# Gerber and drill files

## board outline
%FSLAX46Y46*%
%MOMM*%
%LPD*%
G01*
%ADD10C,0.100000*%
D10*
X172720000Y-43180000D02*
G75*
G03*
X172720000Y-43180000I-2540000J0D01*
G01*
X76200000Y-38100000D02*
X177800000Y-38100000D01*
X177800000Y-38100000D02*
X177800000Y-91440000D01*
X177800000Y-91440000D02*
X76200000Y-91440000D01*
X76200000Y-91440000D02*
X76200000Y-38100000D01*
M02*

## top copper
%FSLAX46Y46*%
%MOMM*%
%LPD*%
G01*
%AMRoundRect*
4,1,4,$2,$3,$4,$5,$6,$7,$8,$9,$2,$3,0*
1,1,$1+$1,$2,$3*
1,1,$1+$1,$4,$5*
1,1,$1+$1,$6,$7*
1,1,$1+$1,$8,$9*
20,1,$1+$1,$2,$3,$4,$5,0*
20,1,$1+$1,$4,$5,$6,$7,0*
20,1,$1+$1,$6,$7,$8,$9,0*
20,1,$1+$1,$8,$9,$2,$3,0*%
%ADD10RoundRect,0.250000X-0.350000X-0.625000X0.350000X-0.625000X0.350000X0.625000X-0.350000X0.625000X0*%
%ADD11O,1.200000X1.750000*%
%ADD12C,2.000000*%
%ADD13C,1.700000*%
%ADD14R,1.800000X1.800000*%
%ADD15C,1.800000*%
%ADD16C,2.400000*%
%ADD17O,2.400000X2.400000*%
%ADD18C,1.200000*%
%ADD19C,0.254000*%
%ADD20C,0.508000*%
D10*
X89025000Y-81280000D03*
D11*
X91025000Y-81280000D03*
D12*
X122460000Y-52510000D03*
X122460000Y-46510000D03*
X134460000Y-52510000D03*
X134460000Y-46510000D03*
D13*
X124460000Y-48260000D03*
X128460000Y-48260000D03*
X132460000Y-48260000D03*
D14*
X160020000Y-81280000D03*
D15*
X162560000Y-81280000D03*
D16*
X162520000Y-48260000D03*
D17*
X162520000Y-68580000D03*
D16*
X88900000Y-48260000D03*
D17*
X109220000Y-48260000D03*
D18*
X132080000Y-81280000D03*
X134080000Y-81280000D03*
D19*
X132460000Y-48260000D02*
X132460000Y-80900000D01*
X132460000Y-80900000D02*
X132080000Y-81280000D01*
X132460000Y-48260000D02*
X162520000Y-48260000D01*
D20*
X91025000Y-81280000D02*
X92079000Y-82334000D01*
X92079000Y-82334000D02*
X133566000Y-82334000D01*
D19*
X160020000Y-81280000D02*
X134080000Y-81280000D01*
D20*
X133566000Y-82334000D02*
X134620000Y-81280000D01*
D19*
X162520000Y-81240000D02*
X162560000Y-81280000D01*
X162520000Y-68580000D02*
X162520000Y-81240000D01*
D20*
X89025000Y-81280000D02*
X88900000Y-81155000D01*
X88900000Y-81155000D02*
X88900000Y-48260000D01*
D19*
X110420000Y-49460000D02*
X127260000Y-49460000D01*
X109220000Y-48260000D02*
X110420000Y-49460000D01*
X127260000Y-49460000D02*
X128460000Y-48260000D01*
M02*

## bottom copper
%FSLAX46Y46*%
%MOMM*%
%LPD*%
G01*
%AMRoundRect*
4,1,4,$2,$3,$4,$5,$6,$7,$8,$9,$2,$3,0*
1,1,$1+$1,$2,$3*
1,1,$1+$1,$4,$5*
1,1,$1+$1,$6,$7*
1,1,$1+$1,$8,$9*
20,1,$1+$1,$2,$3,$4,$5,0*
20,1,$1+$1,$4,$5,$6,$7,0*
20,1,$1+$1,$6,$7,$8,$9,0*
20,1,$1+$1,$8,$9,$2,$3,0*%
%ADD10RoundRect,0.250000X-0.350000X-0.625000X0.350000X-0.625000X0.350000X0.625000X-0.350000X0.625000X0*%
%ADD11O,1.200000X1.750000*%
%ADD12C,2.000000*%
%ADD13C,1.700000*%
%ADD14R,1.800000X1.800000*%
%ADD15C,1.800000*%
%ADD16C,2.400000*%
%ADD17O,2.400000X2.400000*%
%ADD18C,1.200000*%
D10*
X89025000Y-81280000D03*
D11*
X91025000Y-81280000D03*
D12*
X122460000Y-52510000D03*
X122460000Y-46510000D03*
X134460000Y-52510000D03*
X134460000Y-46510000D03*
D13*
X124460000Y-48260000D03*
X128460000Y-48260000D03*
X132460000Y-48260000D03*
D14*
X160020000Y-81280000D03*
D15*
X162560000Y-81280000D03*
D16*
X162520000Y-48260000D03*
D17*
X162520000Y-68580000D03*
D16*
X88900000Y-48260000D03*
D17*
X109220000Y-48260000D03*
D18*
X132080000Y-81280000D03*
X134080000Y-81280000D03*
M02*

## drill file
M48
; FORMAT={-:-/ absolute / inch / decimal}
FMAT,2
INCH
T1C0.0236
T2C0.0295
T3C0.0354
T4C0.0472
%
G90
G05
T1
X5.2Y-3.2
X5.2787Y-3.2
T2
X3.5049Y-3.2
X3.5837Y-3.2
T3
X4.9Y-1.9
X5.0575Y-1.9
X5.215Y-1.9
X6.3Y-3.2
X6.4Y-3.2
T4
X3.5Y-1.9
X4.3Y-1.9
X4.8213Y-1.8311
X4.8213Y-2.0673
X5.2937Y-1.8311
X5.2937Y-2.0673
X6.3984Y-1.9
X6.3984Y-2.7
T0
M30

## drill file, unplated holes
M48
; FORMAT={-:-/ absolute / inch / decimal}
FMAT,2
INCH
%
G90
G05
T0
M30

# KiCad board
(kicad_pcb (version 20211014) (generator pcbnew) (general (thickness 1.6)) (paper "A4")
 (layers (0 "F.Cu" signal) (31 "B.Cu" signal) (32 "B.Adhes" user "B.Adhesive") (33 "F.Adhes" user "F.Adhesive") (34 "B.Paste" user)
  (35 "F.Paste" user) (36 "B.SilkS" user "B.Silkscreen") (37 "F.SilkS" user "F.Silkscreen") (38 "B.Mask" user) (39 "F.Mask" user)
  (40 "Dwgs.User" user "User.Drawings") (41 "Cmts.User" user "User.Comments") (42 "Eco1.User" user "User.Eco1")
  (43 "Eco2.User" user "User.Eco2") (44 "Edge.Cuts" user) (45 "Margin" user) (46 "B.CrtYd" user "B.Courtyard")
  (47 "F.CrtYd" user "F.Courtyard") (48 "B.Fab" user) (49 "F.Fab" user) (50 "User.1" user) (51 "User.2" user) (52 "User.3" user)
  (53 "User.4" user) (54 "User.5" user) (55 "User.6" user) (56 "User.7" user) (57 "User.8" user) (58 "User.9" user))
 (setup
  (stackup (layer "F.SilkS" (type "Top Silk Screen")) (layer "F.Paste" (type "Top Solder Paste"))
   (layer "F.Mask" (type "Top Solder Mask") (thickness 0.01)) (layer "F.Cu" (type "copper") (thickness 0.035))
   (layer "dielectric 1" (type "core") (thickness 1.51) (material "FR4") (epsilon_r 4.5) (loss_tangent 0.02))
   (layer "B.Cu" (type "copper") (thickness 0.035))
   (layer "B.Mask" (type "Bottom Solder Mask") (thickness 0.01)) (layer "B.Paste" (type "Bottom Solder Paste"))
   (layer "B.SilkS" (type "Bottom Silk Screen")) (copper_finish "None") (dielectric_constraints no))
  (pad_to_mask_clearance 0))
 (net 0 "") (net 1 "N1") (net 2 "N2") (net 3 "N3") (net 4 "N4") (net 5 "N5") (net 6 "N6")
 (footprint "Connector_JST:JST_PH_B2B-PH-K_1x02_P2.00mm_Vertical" (layer "F.Cu") (at 89.025 81.28)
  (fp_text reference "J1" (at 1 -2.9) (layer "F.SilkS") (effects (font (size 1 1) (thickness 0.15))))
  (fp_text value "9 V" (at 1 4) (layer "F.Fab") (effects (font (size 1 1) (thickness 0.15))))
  (pad "1" thru_hole roundrect (at 0 0) (size 1.2 1.75) (drill 0.75) (layers *.Cu *.Mask) (roundrect_rratio 0.2083333333) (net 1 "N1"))
  (pad "2" thru_hole oval (at 2 0) (size 1.2 1.75) (drill 0.75) (layers *.Cu *.Mask) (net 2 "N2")))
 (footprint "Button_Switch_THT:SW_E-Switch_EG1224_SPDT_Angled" (layer "F.Cu") (at 124.46 48.26)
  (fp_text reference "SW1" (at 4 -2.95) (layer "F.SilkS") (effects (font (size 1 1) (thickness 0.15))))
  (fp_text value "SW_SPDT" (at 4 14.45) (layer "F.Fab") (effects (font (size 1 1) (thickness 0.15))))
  (pad "" thru_hole circle (at -2 4.25) (size 2 2) (drill 1.2) (layers *.Cu *.Mask))
  (pad "" thru_hole circle (at -2 -1.75) (size 2 2) (drill 1.2) (layers *.Cu *.Mask))
  (pad "" thru_hole circle (at 10 4.25) (size 2 2) (drill 1.2) (layers *.Cu *.Mask))
  (pad "" thru_hole circle (at 10 -1.75) (size 2 2) (drill 1.2) (layers *.Cu *.Mask))
  (pad "1" thru_hole circle (at 0 0) (size 1.7 1.7) (drill 0.9) (layers *.Cu *.Mask) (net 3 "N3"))
  (pad "2" thru_hole circle (at 4 0) (size 1.7 1.7) (drill 0.9) (layers *.Cu *.Mask) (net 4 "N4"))
  (pad "3" thru_hole circle (at 8 0) (size 1.7 1.7) (drill 0.9) (layers *.Cu *.Mask) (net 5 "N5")))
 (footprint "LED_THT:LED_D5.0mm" (layer "F.Cu") (at 160.02 81.28)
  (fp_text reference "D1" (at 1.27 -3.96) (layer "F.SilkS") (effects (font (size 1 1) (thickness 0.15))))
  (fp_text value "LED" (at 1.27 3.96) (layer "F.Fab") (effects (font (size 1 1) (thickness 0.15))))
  (pad "1" thru_hole rect (at 0 0) (size 1.8 1.8) (drill 0.9) (layers *.Cu *.Mask) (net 2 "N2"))
  (pad "2" thru_hole circle (at 2.54 0) (size 1.8 1.8) (drill 0.9) (layers *.Cu *.Mask) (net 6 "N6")))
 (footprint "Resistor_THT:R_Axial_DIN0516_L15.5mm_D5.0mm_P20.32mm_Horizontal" (layer "F.Cu") (at 162.52 48.26 -90)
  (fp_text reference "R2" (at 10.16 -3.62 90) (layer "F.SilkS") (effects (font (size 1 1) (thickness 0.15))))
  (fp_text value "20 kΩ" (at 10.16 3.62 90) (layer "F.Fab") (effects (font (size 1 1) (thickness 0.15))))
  (pad "1" thru_hole circle (at 0 0 270) (size 2.4 2.4) (drill 1.2) (layers *.Cu *.Mask) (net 5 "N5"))
  (pad "2" thru_hole oval (at 20.32 0 270) (size 2.4 2.4) (drill 1.2) (layers *.Cu *.Mask) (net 6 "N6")))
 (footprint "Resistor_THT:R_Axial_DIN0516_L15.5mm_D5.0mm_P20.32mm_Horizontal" (layer "F.Cu") (at 88.9 48.26)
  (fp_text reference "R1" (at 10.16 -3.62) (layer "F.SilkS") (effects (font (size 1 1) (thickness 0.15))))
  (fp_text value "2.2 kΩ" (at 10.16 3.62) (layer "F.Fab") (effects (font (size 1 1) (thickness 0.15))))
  (pad "1" thru_hole circle (at 0 0) (size 2.4 2.4) (drill 1.2) (layers *.Cu *.Mask) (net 1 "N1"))
  (pad "2" thru_hole oval (at 20.32 0) (size 2.4 2.4) (drill 1.2) (layers *.Cu *.Mask) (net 4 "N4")))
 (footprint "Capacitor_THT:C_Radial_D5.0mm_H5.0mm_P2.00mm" (layer "F.Cu") (at 132.08 81.28)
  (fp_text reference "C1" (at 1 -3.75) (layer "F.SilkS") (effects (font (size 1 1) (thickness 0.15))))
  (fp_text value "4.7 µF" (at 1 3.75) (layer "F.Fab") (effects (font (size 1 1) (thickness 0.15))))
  (pad "1" thru_hole circle (at 0 0) (size 1.2 1.2) (drill 0.6) (layers *.Cu *.Mask) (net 5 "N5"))
  (pad "2" thru_hole circle (at 2 0) (size 1.2 1.2) (drill 0.6) (layers *.Cu *.Mask) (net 2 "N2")))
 (gr_circle (center 170.18 43.18) (end 172.72 43.18) (layer "Edge.Cuts") (width 0.1) (fill none))
 (gr_rect (start 76.2 38.1) (end 177.8 91.44) (layer "Edge.Cuts") (width 0.1) (fill none))
 (segment (start 132.46 48.26) (end 132.46 80.9) (width 0.254) (layer "F.Cu") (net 5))
 (segment (start 132.46 80.9) (end 132.08 81.28) (width 0.254) (layer "F.Cu") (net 5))
 (segment (start 132.46 48.26) (end 162.52 48.26) (width 0.254) (layer "F.Cu") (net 5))
 (segment (start 91.025 81.28) (end 92.079 82.334) (width 0.508) (layer "F.Cu") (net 2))
 (segment (start 92.079 82.334) (end 133.566 82.334) (width 0.508) (layer "F.Cu") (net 2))
 (segment (start 160.02 81.28) (end 134.08 81.28) (width 0.254) (layer "F.Cu") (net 2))
 (segment (start 133.566 82.334) (end 134.62 81.28) (width 0.508) (layer "F.Cu") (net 2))
 (segment (start 162.52 81.24) (end 162.56 81.28) (width 0.254) (layer "F.Cu") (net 6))
 (segment (start 162.52 68.58) (end 162.52 81.24) (width 0.254) (layer "F.Cu") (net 6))
 (segment (start 89.025 81.28) (end 88.9 81.155) (width 0.508) (layer "F.Cu") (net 1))
 (segment (start 88.9 81.155) (end 88.9 48.26) (width 0.508) (layer "F.Cu") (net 1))
 (segment (start 110.42 49.46) (end 127.26 49.46) (width 0.254) (layer "F.Cu") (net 4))
 (segment (start 109.22 48.26) (end 110.42 49.46) (width 0.254) (layer "F.Cu") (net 4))
 (segment (start 127.26 49.46) (end 128.46 48.26) (width 0.254) (layer "F.Cu") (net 4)))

